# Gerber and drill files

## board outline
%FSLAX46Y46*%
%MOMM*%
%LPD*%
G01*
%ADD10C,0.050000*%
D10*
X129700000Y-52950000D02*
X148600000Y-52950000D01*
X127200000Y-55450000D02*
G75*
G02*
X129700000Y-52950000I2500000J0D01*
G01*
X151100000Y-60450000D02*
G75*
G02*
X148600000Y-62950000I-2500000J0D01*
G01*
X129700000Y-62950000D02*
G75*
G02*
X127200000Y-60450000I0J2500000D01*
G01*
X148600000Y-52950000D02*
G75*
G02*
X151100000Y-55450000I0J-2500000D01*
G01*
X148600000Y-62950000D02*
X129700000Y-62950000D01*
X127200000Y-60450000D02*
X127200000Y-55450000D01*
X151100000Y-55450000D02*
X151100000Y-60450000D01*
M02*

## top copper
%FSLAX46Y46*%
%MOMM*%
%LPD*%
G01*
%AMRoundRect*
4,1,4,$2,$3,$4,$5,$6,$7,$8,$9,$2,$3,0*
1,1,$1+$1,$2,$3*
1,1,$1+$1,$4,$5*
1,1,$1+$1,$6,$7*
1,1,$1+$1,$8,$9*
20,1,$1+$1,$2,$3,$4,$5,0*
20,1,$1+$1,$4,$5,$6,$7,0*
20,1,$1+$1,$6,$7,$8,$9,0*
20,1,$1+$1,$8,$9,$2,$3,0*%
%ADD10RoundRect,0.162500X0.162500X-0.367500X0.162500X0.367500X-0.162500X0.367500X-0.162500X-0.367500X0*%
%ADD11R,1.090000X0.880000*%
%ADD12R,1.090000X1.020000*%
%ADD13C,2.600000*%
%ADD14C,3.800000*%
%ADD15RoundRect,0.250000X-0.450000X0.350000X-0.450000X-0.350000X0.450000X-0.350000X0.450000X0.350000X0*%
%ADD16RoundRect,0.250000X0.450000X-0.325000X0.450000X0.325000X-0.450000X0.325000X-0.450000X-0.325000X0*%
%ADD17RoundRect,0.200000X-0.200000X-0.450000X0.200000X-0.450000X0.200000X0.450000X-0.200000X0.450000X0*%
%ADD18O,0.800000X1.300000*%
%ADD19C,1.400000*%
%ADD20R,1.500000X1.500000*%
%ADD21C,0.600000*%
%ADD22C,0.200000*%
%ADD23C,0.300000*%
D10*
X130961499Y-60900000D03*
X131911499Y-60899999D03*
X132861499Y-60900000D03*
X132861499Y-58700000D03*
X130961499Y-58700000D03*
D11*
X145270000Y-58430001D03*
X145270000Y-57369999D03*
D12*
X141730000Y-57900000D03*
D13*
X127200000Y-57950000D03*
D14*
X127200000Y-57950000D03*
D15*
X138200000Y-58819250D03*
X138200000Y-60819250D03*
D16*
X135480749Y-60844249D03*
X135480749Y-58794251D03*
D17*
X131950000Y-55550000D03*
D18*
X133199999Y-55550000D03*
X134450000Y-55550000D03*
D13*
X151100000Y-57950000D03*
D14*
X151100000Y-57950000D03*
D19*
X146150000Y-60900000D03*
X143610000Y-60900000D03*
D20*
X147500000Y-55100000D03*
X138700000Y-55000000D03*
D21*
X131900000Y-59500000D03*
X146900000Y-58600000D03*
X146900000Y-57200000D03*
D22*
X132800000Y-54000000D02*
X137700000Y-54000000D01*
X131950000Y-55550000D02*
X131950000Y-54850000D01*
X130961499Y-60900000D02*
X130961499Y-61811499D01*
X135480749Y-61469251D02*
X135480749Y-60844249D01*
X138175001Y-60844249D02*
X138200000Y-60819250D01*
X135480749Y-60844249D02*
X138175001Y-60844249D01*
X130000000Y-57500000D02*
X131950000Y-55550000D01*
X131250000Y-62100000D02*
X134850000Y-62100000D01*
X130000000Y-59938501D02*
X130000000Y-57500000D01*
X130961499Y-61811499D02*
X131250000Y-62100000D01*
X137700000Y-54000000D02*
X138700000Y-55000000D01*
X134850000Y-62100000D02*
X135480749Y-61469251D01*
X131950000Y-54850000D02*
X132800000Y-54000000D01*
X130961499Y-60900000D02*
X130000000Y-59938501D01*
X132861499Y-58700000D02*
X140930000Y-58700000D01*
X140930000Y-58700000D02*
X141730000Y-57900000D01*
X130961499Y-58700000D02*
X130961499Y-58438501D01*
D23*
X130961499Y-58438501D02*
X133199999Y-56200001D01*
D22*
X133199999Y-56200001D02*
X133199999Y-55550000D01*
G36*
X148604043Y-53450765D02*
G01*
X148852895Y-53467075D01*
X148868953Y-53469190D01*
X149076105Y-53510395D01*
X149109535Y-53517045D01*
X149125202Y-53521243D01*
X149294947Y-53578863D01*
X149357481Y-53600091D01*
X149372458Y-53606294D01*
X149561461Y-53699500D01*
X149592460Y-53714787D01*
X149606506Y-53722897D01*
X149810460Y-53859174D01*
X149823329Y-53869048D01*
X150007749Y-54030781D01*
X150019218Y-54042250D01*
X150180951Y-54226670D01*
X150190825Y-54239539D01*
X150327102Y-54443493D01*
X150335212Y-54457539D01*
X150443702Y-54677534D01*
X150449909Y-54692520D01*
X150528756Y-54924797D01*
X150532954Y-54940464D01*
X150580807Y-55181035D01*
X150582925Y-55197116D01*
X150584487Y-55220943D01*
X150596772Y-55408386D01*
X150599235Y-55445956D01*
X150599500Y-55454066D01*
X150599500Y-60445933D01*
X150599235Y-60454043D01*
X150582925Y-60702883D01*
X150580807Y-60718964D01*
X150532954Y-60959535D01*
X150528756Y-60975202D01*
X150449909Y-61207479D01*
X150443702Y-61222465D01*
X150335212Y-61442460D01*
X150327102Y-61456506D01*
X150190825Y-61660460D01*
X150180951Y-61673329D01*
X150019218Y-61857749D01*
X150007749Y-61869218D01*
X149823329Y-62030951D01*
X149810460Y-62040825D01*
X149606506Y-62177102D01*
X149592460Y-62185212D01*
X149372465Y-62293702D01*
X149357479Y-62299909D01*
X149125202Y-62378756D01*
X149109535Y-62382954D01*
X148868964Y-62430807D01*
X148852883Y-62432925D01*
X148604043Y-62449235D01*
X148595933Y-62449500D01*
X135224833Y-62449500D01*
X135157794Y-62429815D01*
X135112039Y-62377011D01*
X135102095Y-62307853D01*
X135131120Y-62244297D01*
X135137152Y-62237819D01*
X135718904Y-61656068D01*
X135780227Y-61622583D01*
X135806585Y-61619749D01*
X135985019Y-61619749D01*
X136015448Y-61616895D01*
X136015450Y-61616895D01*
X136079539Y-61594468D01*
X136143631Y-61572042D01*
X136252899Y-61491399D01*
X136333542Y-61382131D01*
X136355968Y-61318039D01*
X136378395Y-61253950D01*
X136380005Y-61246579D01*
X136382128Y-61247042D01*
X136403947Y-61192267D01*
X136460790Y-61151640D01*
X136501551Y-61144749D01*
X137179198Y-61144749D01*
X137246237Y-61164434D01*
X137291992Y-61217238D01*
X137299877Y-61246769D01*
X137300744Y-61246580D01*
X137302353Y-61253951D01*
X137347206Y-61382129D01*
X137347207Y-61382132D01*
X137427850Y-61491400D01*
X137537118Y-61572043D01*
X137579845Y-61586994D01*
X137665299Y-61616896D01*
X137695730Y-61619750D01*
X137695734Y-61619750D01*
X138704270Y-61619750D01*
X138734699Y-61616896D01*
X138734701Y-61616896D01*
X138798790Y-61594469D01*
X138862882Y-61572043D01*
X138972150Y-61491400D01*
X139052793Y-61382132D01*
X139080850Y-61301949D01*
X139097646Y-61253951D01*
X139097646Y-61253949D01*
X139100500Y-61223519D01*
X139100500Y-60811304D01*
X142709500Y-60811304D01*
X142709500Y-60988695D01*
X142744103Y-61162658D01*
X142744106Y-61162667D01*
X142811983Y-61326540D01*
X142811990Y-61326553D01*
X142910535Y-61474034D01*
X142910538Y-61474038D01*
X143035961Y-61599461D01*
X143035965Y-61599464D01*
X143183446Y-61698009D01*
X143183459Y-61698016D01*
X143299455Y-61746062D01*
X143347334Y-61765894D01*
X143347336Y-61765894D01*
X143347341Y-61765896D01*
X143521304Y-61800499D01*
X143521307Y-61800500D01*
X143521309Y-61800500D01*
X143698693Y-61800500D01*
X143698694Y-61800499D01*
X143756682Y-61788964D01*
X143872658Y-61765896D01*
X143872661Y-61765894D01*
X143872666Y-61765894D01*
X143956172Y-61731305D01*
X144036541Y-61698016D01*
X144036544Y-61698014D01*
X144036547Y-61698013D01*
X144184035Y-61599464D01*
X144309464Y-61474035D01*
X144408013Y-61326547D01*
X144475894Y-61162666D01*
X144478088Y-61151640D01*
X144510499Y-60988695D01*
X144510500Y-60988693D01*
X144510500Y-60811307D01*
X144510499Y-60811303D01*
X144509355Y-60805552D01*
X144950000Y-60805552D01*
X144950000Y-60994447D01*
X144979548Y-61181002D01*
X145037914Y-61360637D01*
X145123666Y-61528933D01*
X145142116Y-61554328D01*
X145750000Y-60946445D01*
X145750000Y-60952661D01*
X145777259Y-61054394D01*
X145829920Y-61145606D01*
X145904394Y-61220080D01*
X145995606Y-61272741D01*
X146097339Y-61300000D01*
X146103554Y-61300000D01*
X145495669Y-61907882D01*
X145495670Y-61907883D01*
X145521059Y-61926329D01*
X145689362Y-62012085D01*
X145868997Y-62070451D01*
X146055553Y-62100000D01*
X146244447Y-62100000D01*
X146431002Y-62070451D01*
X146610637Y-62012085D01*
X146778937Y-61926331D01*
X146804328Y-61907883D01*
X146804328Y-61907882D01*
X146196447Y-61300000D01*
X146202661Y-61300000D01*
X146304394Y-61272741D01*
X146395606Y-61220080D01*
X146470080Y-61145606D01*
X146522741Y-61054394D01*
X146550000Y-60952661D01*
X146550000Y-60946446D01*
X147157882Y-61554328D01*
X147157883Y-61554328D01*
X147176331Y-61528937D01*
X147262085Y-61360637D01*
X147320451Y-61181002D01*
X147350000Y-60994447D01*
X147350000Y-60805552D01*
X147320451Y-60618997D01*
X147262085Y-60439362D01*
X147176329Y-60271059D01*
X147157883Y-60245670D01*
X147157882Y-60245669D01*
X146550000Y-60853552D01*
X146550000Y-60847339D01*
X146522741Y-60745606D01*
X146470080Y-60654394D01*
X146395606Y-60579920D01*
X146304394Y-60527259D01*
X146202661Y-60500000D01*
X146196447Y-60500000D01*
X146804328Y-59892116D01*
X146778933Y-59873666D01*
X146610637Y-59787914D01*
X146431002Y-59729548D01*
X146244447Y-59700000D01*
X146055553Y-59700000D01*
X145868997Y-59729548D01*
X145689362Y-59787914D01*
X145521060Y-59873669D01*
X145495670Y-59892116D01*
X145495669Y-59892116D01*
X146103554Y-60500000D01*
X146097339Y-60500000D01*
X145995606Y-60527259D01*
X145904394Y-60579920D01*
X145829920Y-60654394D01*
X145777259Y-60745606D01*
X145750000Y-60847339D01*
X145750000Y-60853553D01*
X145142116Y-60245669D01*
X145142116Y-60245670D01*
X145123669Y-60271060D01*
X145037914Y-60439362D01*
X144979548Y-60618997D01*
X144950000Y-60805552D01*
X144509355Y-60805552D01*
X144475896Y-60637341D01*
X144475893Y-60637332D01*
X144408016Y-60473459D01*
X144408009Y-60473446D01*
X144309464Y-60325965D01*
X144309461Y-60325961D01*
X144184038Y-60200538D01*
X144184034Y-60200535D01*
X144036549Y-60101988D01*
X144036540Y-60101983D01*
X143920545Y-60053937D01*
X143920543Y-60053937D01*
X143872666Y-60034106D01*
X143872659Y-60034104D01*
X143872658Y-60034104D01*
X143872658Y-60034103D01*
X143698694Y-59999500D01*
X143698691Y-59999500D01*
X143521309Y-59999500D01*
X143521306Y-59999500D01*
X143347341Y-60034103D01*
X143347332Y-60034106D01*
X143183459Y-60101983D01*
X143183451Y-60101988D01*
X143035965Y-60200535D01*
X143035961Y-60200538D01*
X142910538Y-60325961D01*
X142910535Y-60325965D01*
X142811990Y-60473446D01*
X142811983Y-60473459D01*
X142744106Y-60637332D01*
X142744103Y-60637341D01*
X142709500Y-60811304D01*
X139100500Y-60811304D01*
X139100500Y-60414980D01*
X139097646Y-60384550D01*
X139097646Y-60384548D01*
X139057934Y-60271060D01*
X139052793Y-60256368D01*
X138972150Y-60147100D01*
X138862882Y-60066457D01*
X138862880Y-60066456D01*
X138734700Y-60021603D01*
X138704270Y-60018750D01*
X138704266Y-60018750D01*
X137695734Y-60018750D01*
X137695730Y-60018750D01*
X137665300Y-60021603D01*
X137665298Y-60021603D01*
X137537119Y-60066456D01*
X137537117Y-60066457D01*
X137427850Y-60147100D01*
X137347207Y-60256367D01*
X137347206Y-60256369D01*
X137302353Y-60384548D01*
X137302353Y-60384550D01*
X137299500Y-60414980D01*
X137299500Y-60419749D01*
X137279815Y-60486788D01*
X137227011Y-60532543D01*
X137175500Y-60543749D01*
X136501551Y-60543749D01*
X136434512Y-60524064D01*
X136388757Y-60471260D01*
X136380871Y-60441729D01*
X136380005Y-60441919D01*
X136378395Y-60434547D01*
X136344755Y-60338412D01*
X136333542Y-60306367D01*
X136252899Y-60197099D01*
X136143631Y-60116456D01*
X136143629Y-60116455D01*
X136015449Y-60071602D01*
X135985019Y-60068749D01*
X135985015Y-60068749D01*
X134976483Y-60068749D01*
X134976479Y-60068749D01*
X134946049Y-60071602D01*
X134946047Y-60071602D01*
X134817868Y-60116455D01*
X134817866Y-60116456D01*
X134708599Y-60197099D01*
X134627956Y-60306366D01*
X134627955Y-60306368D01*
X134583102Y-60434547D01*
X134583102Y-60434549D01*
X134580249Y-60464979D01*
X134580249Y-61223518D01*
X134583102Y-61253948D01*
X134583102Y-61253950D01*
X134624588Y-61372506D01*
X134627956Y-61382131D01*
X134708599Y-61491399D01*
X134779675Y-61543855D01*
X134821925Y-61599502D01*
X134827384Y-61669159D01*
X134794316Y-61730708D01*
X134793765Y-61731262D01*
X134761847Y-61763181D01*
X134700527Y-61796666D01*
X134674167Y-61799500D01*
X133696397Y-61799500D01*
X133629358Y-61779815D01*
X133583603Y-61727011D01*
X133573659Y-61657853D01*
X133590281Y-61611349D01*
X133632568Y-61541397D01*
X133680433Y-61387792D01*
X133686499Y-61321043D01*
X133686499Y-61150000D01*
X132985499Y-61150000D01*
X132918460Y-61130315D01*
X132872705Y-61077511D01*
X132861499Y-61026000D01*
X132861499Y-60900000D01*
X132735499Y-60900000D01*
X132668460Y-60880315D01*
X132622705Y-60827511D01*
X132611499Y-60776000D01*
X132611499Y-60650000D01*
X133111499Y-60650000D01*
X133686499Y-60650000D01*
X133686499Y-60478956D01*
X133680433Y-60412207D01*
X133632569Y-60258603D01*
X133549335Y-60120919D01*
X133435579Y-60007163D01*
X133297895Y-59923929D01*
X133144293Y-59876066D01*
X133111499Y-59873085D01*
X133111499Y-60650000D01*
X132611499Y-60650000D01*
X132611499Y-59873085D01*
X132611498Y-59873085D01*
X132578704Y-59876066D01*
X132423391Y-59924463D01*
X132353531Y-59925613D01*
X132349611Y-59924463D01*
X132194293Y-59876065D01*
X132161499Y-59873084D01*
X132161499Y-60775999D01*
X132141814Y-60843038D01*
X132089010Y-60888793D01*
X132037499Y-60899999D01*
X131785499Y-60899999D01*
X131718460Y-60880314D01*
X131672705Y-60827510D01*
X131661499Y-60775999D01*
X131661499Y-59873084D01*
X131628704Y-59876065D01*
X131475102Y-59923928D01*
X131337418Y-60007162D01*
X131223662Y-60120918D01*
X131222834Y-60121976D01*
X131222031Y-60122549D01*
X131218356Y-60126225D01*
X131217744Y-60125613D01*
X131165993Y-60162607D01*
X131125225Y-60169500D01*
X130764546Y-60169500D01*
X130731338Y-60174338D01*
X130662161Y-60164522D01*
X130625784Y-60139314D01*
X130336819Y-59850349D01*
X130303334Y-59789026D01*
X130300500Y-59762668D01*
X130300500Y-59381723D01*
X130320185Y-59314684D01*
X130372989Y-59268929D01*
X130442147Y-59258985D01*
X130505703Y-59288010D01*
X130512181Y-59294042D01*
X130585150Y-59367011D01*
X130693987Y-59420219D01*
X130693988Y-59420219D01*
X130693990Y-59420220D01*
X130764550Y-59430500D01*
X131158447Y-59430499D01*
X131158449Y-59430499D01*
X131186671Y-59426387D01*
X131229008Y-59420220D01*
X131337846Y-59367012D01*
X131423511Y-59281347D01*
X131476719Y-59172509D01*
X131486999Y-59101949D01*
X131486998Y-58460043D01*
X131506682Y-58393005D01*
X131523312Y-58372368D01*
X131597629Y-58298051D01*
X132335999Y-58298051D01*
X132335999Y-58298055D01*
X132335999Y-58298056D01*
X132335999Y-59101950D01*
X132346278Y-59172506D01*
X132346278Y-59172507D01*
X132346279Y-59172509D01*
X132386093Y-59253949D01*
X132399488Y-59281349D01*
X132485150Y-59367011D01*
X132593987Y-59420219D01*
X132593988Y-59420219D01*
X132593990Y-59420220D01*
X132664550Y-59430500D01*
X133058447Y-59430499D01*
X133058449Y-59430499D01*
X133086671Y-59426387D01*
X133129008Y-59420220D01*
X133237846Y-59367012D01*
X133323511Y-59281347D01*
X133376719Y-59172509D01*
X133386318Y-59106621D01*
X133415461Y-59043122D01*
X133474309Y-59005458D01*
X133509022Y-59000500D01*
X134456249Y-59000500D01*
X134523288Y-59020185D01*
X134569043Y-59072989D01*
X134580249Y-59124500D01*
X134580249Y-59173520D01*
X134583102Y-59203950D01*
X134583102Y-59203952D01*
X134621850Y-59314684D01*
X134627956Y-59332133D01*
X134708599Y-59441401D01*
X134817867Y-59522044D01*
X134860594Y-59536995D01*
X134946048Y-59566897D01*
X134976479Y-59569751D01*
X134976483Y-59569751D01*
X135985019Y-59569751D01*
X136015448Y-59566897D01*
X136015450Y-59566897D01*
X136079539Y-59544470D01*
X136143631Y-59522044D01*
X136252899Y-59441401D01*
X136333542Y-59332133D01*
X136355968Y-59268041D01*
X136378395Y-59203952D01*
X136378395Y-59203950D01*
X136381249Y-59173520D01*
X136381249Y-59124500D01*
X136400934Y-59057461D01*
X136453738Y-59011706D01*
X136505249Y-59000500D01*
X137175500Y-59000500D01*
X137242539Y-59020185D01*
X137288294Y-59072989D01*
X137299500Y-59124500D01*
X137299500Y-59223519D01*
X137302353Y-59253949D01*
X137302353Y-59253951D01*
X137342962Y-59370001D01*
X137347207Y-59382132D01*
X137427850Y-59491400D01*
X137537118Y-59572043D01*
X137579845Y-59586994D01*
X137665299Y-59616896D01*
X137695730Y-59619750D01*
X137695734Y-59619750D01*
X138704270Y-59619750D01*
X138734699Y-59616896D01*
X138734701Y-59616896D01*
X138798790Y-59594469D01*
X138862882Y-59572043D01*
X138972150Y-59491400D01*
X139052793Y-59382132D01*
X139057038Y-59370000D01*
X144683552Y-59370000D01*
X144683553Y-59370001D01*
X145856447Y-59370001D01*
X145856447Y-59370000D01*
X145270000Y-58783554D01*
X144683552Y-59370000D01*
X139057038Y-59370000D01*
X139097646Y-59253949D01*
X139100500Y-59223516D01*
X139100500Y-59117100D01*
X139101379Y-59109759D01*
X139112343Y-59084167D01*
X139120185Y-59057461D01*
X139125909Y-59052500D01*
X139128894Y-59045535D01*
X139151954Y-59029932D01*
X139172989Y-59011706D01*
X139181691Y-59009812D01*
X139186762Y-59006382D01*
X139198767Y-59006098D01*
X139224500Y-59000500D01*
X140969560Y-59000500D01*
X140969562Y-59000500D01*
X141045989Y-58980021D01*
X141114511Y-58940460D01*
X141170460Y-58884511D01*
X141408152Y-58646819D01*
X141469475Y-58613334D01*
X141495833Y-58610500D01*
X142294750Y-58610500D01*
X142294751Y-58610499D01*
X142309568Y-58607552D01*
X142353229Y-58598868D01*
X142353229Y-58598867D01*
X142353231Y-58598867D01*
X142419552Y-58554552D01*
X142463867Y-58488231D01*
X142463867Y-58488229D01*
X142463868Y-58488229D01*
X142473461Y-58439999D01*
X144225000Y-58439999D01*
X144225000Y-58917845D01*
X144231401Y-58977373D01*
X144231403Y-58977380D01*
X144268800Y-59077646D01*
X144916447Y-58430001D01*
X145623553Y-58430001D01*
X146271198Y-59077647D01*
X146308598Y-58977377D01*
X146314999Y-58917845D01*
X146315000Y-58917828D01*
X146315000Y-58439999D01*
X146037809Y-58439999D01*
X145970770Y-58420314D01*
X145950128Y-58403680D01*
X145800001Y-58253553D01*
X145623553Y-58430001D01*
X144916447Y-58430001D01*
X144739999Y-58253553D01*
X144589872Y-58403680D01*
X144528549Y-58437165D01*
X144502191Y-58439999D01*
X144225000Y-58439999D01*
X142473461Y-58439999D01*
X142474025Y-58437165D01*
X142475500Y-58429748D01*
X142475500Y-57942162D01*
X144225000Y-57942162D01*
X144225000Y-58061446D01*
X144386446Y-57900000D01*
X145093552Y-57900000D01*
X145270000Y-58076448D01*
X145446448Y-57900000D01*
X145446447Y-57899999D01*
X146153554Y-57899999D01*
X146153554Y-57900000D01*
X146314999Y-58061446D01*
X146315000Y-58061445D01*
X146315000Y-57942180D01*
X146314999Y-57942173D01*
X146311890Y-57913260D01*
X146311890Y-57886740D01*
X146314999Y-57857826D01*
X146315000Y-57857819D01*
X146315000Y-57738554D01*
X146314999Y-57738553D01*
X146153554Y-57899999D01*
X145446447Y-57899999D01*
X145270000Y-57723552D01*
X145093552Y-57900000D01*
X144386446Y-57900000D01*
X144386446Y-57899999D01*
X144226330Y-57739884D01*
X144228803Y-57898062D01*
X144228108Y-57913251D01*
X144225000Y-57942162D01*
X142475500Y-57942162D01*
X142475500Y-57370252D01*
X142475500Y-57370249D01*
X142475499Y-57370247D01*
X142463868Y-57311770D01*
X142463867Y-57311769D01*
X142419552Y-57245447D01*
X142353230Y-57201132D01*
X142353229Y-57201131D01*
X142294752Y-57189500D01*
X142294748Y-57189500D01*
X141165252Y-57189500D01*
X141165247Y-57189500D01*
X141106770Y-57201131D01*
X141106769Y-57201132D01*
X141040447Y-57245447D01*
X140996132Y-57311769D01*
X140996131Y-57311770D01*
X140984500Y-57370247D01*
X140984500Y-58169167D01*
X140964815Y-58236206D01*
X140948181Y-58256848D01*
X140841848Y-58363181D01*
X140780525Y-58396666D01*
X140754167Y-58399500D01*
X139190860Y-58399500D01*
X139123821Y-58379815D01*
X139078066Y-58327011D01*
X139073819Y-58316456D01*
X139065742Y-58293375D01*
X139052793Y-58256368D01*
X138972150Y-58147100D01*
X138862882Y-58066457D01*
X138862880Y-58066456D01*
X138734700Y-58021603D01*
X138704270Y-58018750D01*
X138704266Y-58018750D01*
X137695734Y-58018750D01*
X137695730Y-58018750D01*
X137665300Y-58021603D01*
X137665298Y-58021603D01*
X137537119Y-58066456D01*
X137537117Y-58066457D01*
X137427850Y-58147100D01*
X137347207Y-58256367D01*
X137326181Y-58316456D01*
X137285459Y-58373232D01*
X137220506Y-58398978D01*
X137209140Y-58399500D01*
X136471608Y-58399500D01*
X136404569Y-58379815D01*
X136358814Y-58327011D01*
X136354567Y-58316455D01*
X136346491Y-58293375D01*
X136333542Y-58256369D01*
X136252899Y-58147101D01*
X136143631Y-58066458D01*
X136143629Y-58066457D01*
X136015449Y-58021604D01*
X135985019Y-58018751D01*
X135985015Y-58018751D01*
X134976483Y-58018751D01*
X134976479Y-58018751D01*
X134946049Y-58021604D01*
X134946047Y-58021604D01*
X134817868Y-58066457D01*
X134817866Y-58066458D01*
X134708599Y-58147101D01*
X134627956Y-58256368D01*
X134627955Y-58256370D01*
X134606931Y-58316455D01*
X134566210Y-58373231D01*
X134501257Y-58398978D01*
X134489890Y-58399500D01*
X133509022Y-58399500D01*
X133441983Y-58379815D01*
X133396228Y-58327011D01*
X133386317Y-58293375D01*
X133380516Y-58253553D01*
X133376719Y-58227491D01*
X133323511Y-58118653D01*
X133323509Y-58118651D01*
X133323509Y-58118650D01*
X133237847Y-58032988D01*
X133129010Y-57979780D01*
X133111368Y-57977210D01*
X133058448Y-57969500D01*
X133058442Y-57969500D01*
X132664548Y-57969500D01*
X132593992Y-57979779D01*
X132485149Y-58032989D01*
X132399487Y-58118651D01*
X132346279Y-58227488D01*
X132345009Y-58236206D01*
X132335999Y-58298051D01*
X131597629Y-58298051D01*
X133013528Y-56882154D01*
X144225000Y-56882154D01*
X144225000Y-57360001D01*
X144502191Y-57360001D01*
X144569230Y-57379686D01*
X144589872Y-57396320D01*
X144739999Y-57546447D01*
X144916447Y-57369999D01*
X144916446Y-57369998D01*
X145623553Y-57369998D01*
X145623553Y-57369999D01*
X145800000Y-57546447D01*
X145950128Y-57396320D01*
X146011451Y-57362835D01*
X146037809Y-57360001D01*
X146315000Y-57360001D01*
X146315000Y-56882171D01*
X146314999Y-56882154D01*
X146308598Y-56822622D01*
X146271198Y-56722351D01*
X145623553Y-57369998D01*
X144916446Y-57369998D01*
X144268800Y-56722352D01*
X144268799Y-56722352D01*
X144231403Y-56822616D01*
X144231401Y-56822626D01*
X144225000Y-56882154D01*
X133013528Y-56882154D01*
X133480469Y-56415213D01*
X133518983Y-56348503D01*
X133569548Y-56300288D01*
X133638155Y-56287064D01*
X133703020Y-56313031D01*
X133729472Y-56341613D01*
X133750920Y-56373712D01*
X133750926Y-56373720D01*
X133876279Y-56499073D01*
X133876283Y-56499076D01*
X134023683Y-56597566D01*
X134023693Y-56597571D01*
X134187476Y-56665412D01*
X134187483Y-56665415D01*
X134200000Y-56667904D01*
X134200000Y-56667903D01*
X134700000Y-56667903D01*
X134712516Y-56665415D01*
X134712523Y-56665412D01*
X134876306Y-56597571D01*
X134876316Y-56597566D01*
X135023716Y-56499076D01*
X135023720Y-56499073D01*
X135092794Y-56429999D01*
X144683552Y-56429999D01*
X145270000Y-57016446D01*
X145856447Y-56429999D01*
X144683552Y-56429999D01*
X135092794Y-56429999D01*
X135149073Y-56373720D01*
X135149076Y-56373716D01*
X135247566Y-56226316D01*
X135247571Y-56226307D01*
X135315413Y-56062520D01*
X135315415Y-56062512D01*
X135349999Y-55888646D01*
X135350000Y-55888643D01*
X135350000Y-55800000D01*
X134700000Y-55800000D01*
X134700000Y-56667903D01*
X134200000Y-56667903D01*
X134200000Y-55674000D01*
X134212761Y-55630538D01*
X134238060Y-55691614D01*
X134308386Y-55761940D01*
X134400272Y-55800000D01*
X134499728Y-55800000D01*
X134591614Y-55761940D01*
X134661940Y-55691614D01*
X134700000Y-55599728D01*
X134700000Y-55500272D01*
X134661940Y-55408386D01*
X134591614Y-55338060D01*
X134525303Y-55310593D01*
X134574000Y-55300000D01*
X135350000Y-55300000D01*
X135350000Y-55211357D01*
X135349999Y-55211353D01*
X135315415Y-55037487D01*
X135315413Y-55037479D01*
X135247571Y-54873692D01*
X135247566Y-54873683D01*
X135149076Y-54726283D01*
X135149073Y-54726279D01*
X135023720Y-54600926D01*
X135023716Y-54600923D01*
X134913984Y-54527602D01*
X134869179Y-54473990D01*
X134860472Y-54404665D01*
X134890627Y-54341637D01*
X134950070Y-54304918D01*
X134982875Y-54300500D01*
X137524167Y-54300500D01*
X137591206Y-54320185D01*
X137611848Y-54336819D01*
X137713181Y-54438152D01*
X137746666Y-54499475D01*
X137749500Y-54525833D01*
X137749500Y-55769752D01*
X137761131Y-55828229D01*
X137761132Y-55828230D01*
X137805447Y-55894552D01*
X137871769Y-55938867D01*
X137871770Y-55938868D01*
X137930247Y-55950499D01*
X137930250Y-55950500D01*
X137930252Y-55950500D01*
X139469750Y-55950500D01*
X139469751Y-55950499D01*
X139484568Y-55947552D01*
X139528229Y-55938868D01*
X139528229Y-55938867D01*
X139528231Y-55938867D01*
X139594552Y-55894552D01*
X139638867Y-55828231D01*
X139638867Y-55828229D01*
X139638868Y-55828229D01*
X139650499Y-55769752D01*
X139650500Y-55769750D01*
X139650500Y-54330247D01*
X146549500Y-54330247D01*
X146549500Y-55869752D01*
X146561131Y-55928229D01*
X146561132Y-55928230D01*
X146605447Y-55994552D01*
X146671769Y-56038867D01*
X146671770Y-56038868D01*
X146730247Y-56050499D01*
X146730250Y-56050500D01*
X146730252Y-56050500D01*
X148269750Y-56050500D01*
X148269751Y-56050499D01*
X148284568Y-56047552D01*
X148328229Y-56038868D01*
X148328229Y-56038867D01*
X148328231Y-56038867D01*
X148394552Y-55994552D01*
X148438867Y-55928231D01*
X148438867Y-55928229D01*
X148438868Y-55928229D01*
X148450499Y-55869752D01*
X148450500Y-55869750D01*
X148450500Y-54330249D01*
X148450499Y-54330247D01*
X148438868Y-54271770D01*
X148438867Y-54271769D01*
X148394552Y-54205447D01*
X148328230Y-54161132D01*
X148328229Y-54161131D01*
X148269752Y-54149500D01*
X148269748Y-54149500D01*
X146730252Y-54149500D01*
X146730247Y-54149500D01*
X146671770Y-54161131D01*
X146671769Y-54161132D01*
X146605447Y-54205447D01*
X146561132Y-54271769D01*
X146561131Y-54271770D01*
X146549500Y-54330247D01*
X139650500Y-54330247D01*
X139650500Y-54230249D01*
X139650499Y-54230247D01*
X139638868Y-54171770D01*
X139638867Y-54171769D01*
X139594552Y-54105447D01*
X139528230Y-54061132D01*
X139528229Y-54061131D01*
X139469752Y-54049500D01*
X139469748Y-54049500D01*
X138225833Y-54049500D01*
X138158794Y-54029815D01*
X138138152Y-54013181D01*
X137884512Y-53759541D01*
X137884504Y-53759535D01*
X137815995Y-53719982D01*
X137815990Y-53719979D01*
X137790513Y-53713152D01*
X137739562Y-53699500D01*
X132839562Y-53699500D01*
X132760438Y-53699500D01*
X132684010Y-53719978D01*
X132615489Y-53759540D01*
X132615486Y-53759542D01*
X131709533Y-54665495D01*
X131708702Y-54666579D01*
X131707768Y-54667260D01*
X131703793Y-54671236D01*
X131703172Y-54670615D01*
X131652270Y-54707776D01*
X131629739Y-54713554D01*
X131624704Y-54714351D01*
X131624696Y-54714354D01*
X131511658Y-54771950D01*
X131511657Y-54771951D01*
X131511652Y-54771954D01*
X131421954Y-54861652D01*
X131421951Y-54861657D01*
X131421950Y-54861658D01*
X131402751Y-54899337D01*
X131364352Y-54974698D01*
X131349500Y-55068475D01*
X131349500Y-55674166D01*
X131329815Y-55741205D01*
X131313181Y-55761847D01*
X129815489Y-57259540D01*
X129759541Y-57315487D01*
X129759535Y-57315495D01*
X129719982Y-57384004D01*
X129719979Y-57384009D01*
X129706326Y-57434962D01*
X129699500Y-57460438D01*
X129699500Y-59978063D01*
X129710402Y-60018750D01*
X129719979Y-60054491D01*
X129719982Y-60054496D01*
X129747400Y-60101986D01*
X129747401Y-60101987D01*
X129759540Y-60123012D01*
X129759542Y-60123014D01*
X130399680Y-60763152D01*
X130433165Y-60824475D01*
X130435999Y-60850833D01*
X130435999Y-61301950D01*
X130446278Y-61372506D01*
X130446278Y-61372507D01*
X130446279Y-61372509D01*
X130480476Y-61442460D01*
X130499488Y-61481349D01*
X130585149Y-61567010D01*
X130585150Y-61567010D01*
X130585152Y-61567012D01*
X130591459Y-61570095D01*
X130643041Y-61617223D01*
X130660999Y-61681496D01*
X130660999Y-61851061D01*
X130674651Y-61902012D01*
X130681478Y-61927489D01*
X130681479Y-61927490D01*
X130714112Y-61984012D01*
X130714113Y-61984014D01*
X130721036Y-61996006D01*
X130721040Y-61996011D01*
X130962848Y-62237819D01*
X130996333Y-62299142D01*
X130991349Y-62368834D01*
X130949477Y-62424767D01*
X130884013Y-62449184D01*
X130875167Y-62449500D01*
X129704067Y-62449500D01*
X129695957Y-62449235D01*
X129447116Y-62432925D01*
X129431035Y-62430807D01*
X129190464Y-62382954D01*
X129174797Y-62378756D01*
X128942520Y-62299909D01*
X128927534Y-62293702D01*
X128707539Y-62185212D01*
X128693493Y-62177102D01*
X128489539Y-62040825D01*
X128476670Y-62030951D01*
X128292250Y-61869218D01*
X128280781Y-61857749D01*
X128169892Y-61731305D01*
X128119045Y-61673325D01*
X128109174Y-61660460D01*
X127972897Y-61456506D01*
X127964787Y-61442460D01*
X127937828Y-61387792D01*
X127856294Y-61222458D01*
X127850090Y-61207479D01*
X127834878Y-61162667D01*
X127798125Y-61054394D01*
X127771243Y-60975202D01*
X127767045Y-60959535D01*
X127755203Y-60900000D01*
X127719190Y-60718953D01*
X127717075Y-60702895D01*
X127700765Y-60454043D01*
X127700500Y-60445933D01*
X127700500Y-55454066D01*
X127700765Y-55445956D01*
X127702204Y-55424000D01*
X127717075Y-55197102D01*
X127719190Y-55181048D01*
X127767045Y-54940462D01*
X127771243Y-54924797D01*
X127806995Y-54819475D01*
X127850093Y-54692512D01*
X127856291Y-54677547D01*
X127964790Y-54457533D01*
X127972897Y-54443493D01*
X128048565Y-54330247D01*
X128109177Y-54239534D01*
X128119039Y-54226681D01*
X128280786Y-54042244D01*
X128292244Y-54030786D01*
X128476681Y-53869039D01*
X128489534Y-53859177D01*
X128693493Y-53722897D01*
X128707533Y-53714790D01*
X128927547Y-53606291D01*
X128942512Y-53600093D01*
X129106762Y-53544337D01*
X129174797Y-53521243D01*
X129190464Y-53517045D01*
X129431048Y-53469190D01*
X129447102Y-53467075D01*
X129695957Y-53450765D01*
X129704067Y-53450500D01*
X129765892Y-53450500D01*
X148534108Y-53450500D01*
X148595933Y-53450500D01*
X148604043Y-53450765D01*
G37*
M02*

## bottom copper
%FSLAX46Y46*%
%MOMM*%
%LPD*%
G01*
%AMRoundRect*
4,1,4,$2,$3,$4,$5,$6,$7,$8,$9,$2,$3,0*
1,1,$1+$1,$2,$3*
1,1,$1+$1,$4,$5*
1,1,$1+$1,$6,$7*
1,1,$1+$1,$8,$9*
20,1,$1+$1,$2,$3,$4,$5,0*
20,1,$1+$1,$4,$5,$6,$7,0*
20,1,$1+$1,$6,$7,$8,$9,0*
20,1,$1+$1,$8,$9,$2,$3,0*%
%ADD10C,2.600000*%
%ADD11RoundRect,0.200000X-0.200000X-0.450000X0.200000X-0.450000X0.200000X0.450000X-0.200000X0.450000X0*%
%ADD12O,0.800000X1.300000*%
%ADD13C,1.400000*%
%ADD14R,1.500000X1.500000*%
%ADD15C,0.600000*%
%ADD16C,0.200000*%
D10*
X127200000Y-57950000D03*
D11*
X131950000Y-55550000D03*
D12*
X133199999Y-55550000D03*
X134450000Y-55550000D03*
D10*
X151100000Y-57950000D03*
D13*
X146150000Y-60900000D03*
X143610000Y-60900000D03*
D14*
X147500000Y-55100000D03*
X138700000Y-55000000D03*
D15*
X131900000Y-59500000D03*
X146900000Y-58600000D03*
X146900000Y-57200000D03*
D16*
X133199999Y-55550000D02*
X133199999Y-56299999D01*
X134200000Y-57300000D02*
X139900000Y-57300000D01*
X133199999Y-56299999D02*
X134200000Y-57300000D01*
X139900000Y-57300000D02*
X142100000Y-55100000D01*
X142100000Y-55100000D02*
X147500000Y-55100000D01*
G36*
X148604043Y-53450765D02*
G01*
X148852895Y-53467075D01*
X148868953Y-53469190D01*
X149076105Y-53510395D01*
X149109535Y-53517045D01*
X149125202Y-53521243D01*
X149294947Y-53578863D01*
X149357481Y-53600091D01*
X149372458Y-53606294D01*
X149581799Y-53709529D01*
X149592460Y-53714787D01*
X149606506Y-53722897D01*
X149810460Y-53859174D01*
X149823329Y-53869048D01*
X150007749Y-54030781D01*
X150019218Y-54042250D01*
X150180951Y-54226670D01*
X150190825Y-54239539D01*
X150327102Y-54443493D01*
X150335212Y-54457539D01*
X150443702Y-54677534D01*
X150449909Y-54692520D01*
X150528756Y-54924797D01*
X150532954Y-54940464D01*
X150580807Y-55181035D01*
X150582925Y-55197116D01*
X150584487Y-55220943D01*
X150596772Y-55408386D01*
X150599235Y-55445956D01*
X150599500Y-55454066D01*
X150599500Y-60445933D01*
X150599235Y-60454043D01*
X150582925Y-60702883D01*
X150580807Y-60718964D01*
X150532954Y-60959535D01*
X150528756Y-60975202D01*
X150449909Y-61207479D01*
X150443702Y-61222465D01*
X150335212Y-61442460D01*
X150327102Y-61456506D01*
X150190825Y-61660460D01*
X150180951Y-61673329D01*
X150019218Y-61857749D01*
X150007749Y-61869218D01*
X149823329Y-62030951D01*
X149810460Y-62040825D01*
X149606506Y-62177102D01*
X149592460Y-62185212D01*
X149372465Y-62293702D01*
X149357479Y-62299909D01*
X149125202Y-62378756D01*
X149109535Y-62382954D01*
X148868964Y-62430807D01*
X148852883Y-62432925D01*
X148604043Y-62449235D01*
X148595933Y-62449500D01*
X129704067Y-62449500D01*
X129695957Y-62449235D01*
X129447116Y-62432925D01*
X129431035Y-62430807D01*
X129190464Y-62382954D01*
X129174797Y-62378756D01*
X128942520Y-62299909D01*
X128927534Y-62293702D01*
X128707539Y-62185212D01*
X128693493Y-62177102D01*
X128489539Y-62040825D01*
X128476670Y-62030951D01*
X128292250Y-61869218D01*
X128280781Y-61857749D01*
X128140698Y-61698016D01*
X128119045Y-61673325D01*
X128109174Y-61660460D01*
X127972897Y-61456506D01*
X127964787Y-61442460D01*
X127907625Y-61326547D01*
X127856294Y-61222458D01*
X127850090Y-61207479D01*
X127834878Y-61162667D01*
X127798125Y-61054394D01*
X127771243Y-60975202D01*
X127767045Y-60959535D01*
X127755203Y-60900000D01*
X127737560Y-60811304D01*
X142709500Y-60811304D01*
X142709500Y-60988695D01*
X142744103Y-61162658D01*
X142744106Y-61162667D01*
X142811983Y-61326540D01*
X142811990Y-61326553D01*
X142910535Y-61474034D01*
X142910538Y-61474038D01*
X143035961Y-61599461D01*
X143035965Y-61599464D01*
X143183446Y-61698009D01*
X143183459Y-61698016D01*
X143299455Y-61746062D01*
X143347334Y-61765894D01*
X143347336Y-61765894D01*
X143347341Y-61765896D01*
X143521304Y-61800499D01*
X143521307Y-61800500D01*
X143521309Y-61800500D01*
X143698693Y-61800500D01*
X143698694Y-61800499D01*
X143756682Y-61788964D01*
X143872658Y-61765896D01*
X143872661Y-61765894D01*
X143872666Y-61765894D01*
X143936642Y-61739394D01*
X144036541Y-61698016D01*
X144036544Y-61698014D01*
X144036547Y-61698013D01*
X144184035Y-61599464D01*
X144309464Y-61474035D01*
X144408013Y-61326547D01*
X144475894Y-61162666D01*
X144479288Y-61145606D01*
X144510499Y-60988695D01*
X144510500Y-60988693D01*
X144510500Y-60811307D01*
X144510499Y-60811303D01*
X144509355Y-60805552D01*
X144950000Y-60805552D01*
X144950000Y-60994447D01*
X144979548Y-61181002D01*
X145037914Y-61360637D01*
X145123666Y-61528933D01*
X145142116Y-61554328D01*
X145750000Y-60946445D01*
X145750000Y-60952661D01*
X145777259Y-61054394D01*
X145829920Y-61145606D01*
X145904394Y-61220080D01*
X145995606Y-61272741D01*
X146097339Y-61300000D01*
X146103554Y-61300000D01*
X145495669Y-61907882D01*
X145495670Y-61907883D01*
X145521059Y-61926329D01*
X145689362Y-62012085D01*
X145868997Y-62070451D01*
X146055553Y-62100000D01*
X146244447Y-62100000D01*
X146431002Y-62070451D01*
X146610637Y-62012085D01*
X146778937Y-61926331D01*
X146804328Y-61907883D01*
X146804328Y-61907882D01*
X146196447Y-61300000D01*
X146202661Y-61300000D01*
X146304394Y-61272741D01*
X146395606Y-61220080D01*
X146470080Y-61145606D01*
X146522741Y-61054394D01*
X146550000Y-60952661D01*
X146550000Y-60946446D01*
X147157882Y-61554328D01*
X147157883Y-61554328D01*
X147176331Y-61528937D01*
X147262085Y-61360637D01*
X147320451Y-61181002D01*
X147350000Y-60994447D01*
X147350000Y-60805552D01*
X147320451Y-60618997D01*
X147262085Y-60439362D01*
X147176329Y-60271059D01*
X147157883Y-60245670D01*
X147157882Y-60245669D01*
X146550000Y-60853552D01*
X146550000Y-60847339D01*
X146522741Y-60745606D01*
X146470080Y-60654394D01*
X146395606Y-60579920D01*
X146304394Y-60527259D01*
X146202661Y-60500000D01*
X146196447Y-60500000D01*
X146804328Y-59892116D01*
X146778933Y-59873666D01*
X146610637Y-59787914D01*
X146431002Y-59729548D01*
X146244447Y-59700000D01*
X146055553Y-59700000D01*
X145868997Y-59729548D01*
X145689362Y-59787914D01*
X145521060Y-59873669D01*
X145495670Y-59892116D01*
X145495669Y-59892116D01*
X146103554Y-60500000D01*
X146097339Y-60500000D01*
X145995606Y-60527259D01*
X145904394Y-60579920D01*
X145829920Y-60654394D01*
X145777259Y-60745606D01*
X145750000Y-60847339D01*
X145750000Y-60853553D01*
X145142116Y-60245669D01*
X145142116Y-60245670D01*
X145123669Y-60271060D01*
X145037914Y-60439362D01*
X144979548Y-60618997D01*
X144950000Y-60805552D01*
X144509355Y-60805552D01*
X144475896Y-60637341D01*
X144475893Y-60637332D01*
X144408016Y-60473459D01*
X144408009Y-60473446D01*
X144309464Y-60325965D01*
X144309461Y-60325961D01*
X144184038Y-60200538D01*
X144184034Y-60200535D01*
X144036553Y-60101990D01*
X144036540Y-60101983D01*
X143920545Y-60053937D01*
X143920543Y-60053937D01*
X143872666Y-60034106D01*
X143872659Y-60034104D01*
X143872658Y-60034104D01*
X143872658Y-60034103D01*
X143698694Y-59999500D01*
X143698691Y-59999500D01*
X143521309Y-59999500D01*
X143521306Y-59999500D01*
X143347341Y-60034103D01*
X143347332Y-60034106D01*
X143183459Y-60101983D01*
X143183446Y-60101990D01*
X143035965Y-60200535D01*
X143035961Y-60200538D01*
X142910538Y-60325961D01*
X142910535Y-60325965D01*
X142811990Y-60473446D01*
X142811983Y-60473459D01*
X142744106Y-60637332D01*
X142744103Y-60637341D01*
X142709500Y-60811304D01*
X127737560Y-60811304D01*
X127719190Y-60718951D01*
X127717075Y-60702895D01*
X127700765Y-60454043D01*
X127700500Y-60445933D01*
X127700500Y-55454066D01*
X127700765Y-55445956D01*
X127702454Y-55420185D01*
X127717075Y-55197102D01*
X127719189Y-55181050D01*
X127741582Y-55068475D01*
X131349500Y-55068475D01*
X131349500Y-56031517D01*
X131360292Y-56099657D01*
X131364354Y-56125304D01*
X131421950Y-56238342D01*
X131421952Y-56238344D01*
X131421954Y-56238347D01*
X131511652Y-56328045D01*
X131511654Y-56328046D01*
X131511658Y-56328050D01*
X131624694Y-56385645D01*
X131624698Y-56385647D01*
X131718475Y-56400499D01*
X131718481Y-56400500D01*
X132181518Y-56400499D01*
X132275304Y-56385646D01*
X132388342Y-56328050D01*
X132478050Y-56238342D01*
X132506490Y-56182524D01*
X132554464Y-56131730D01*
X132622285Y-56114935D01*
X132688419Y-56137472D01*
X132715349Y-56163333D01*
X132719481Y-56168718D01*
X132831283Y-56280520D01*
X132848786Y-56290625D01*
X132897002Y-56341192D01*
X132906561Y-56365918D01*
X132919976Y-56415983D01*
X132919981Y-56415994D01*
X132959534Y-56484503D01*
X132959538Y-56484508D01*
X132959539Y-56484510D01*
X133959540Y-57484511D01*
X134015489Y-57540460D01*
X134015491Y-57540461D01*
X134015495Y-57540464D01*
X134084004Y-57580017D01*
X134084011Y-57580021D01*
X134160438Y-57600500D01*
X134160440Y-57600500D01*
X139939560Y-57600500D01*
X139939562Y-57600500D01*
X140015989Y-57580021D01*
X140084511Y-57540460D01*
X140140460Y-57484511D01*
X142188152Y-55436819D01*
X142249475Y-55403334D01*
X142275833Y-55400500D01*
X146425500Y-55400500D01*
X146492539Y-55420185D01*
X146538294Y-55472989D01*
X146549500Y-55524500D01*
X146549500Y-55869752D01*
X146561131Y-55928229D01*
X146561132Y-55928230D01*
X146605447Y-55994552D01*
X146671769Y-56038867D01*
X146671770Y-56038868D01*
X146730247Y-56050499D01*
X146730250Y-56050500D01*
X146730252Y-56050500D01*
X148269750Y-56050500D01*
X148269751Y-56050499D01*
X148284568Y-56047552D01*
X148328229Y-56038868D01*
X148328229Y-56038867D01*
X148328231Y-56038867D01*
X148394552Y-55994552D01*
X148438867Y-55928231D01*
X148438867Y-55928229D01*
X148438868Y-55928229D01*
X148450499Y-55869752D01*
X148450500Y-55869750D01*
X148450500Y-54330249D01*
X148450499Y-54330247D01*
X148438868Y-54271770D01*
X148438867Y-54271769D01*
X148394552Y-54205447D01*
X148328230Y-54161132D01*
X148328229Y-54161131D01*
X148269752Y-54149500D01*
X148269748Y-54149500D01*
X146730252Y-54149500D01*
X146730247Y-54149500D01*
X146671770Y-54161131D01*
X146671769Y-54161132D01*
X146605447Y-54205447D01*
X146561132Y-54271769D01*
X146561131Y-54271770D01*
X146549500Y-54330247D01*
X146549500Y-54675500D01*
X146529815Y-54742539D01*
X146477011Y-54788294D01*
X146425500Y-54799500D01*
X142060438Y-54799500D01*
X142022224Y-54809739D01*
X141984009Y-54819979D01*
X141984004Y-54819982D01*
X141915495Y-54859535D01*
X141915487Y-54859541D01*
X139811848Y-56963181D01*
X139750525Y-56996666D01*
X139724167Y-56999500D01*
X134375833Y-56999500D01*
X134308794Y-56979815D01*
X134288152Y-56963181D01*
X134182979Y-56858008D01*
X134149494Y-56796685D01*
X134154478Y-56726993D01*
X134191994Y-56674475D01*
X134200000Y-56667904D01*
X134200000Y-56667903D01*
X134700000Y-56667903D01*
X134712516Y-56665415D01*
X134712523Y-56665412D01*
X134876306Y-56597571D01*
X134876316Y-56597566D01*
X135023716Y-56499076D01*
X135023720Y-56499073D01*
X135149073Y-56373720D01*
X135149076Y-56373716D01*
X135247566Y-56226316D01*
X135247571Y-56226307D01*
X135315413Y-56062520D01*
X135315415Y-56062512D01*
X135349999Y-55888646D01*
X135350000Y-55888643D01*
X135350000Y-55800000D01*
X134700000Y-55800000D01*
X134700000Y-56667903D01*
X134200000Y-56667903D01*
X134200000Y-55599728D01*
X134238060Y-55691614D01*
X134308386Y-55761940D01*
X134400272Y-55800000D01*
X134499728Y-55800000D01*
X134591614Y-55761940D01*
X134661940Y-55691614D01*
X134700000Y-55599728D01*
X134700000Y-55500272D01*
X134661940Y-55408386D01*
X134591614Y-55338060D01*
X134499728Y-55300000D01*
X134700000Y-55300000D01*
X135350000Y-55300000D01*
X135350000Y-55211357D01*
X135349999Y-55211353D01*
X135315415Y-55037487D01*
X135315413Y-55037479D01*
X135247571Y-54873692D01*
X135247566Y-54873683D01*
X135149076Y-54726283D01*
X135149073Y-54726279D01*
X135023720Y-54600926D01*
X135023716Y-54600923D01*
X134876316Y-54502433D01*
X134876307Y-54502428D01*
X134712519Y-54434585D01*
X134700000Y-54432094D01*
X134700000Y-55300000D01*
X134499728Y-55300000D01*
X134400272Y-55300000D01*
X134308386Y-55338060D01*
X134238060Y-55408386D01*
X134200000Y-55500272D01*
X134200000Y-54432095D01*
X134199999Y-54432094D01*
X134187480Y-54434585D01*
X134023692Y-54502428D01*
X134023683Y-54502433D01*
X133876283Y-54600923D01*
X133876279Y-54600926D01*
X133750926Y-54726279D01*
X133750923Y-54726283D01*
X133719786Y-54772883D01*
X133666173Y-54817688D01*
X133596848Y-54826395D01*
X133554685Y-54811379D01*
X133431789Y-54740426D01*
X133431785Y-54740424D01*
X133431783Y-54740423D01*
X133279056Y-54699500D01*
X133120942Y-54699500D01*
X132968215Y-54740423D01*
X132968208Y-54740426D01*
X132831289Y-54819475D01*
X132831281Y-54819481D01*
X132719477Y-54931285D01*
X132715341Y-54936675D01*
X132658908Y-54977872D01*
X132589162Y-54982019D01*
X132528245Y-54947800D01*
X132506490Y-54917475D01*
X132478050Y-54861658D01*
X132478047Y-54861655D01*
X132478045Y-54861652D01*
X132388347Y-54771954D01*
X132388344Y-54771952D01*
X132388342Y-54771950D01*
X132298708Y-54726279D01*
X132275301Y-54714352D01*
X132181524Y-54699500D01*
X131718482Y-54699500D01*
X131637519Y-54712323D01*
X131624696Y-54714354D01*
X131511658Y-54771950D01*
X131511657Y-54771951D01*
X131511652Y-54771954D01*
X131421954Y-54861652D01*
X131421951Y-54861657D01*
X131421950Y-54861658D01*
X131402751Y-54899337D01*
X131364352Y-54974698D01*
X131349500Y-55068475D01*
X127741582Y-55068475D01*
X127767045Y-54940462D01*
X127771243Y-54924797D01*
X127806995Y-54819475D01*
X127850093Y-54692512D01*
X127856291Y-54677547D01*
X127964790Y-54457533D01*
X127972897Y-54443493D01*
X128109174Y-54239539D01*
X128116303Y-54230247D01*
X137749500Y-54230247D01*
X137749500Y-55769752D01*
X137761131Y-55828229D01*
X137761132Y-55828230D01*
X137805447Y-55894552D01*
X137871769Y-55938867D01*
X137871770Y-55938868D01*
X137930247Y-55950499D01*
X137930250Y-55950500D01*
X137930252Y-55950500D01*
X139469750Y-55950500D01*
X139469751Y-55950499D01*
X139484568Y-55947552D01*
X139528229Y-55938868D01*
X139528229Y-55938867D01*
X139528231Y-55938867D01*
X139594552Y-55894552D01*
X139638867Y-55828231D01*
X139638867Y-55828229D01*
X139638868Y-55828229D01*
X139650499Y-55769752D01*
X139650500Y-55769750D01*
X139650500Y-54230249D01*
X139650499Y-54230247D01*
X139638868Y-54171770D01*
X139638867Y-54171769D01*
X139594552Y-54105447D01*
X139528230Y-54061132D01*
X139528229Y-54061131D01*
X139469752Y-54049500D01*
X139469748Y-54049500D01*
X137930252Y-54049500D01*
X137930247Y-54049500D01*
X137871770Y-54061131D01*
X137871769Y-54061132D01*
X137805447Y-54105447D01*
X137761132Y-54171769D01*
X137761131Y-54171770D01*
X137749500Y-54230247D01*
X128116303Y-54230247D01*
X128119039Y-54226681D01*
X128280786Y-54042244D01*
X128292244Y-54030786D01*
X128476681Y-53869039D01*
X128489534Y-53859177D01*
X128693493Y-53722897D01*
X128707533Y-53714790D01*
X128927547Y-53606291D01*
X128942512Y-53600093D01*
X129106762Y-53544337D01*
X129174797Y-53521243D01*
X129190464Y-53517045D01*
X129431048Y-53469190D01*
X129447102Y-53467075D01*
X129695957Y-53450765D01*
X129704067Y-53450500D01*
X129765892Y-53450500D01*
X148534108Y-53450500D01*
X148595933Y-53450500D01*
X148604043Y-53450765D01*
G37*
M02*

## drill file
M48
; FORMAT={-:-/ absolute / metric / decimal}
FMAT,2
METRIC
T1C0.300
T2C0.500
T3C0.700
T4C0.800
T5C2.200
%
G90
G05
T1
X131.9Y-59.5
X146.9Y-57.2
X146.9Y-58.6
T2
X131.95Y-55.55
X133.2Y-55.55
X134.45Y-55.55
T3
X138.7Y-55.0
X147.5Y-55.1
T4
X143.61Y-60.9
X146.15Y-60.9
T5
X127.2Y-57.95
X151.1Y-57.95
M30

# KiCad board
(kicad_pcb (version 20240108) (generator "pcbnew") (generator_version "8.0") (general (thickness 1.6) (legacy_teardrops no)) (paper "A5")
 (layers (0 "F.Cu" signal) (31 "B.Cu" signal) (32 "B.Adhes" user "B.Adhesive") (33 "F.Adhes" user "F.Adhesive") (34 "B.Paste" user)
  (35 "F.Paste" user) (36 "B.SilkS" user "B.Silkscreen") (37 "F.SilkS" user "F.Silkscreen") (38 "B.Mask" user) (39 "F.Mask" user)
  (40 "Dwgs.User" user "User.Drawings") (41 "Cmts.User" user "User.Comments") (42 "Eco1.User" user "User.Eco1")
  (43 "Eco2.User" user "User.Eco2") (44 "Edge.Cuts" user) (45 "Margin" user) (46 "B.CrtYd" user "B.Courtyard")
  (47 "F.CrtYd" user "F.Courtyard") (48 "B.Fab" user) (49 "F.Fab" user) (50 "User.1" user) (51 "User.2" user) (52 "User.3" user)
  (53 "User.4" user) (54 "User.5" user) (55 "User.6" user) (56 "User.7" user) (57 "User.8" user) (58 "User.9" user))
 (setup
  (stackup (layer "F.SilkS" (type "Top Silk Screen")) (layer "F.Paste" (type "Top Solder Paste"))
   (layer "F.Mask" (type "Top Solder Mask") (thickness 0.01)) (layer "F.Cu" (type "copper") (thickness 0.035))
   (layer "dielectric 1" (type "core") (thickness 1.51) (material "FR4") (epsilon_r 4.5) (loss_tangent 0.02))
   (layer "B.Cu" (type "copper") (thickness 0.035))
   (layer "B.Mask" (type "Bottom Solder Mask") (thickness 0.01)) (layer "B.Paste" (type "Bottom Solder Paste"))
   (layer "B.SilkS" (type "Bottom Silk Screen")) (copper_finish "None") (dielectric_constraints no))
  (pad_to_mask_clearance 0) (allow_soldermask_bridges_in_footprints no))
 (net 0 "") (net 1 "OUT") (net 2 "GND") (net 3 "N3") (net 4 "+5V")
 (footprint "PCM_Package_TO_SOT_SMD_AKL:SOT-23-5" (layer "F.Cu") (at 131.911499 59.8 90)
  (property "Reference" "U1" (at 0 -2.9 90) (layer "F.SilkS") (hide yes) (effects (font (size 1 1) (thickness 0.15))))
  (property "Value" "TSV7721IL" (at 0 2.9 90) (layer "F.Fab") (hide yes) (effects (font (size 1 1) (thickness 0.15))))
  (pad "1" smd roundrect (at -1.1 -0.95 90) (size 1.06 0.65) (layers "F.Cu" "F.Paste" "F.Mask") (roundrect_rratio 0.25) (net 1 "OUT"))
  (pad "2" smd roundrect (at -1.099999 0 90) (size 1.06 0.65) (layers "F.Cu" "F.Paste" "F.Mask") (roundrect_rratio 0.25) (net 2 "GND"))
  (pad "3" smd roundrect (at -1.1 0.95 90) (size 1.06 0.65) (layers "F.Cu" "F.Paste" "F.Mask") (roundrect_rratio 0.25) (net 2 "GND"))
  (pad "4" smd roundrect (at 1.1 0.95 90) (size 1.06 0.65) (layers "F.Cu" "F.Paste" "F.Mask") (roundrect_rratio 0.25) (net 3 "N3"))
  (pad "5" smd roundrect (at 1.1 -0.95 90) (size 1.06 0.65) (layers "F.Cu" "F.Paste" "F.Mask") (roundrect_rratio 0.25) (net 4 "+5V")))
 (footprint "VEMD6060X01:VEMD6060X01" (layer "F.Cu") (at 143.5 57.9 180)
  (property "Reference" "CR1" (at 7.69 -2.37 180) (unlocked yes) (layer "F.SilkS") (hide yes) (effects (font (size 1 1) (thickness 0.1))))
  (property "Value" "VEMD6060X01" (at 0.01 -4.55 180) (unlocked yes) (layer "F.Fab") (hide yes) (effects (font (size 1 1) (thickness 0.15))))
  (pad "1" smd rect (at -1.77 -0.530001 180) (size 1.09 0.88) (layers "F.Cu" "F.Paste" "F.Mask") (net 2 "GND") (thermal_bridge_angle 45))
  (pad "2" smd rect (at -1.77 0.530001 180) (size 1.09 0.88) (layers "F.Cu" "F.Paste" "F.Mask") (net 2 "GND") (thermal_bridge_angle 45))
  (pad "3" smd rect (at 1.77 0 180) (size 1.09 1.02) (layers "F.Cu" "F.Paste" "F.Mask") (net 3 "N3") (thermal_bridge_angle 45)))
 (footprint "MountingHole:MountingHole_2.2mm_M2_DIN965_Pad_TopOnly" (layer "F.Cu") (at 127.2 57.95)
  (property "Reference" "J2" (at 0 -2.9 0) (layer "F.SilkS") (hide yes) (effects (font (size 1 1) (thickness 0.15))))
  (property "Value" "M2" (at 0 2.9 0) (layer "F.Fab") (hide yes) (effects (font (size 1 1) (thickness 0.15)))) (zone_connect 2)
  (pad "1" thru_hole circle (at 0 0) (size 2.6 2.6) (drill 2.2) (layers "*.Cu" "*.Mask") (remove_unused_layers no) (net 2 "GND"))
  (pad "1" connect circle (at 0 0) (size 3.8 3.8) (layers "F.Cu" "F.Mask") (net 2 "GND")))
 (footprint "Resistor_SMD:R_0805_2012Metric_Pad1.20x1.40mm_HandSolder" (layer "F.Cu") (at 138.2 59.81925 -90)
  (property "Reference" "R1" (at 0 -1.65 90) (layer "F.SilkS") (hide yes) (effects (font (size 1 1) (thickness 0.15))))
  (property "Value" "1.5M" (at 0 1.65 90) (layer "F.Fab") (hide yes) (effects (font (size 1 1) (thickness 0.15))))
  (pad "1" smd roundrect (at -1 0 270) (size 1.2 1.4) (layers "F.Cu" "F.Paste" "F.Mask") (roundrect_rratio 0.208333) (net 3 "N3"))
  (pad "2" smd roundrect (at 1 0 270) (size 1.2 1.4) (layers "F.Cu" "F.Paste" "F.Mask") (roundrect_rratio 0.208333) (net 1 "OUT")))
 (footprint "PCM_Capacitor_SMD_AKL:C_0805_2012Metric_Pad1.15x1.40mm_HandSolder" (layer "F.Cu") (at 135.480749 59.81925 90)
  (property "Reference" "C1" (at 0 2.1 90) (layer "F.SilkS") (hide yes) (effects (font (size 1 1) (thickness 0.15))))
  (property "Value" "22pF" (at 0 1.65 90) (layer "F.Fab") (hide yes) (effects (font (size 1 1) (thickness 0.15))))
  (pad "1" smd roundrect (at -1.024999 0 90) (size 1.15 1.4) (layers "F.Cu" "F.Paste" "F.Mask") (roundrect_rratio 0.217391) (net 1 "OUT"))
  (pad "2" smd roundrect (at 1.024999 0 90) (size 1.15 1.4) (layers "F.Cu" "F.Paste" "F.Mask") (roundrect_rratio 0.217391) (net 3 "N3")))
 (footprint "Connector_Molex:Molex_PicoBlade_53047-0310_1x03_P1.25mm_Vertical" (layer "F.Cu") (at 131.95 55.55)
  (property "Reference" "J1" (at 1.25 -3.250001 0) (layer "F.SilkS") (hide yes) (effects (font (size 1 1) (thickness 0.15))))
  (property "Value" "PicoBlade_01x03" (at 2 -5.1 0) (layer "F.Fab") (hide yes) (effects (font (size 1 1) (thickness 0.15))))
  (pad "1" thru_hole roundrect (at 0 0) (size 0.8 1.3) (drill 0.5) (layers "*.Cu" "*.Mask") (remove_unused_layers no)
   (roundrect_rratio 0.25) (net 1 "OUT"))
  (pad "2" thru_hole oval (at 1.249999 0) (size 0.8 1.3) (drill 0.5) (layers "*.Cu" "*.Mask") (remove_unused_layers no) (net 4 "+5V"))
  (pad "3" thru_hole oval (at 2.5 0) (size 0.8 1.3) (drill 0.5) (layers "*.Cu" "*.Mask") (remove_unused_layers no) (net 2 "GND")))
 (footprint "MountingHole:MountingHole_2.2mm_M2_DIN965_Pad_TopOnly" (layer "F.Cu") (at 151.1 57.95)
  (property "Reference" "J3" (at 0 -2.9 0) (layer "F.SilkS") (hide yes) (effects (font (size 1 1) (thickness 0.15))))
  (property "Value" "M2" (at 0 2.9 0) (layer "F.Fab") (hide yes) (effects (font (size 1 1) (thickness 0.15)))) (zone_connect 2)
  (pad "1" thru_hole circle (at 0 0) (size 2.6 2.6) (drill 2.2) (layers "*.Cu" "*.Mask") (remove_unused_layers no) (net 2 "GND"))
  (pad "1" connect circle (at 0 0) (size 3.8 3.8) (layers "F.Cu" "F.Mask") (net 2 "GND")))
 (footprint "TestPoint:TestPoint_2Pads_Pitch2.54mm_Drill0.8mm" (layer "B.Cu") (at 146.15 60.9 180)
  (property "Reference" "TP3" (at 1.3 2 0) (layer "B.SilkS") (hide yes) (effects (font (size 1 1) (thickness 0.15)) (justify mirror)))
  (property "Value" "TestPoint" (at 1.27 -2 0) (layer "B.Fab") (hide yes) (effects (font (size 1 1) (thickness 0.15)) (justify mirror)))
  (pad "1" thru_hole circle (at 0 0 180) (size 1.4 1.4) (drill 0.8) (layers "*.Cu" "*.Mask") (remove_unused_layers no) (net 2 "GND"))
  (pad "2" thru_hole circle (at 2.54 0 180) (size 1.4 1.4) (drill 0.8) (layers "*.Cu" "*.Mask") (remove_unused_layers no)))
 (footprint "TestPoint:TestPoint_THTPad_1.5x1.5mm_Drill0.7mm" (layer "B.Cu") (at 147.5 55.1 180)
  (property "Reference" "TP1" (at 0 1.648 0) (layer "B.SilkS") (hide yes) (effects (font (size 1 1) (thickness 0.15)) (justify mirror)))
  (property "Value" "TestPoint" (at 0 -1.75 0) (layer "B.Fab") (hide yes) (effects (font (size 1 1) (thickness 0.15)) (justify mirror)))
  (pad "1" thru_hole rect (at 0 0 180) (size 1.5 1.5) (drill 0.7) (layers "*.Cu" "*.Mask") (remove_unused_layers no) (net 4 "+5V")))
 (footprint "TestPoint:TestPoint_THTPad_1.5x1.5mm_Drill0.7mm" (layer "B.Cu") (at 138.7 55 180)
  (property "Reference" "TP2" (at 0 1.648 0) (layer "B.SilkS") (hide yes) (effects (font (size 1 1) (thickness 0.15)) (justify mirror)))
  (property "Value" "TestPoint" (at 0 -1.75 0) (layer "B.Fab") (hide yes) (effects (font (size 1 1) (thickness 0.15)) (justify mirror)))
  (pad "1" thru_hole rect (at 0 0 180) (size 1.5 1.5) (drill 0.7) (layers "*.Cu" "*.Mask") (remove_unused_layers no) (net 1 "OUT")))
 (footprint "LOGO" (layer "B.Cu") (at 139.13435 57.9 180)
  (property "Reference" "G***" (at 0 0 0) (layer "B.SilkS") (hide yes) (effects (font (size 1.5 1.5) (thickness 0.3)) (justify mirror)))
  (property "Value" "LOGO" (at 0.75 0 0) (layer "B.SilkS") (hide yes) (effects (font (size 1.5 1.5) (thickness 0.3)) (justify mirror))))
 (gr_line (start 129.7 52.95) (end 148.6 52.95) (stroke (width 0.05) (type default)) (layer "Edge.Cuts"))
 (gr_arc (start 127.2 55.45) (mid 127.932233 53.682233) (end 129.7 52.95) (stroke (width 0.05) (type default)) (layer "Edge.Cuts"))
 (gr_arc (start 151.1 60.45) (mid 150.367767 62.217767) (end 148.6 62.95) (stroke (width 0.05) (type default)) (layer "Edge.Cuts"))
 (gr_arc (start 129.7 62.95) (mid 127.932233 62.217767) (end 127.2 60.45) (stroke (width 0.05) (type default)) (layer "Edge.Cuts"))
 (gr_arc (start 148.6 52.95) (mid 150.367767 53.682233) (end 151.1 55.45) (stroke (width 0.05) (type default)) (layer "Edge.Cuts"))
 (gr_line (start 148.6 62.95) (end 129.7 62.95) (stroke (width 0.05) (type default)) (layer "Edge.Cuts"))
 (gr_line (start 127.2 60.45) (end 127.2 55.45) (stroke (width 0.05) (type default)) (layer "Edge.Cuts"))
 (gr_line (start 151.1 55.45) (end 151.1 60.45) (stroke (width 0.05) (type default)) (layer "Edge.Cuts"))
 (segment (start 132.8 54) (end 137.7 54) (width 0.2) (layer "F.Cu") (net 1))
 (segment (start 131.95 55.55) (end 131.95 54.85) (width 0.2) (layer "F.Cu") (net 1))
 (segment (start 130.961499 60.9) (end 130.961499 61.811499) (width 0.2) (layer "F.Cu") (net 1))
 (segment (start 135.480749 61.469251) (end 135.480749 60.844249) (width 0.2) (layer "F.Cu") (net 1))
 (segment (start 138.175001 60.844249) (end 138.2 60.81925) (width 0.2) (layer "F.Cu") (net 1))
 (segment (start 135.480749 60.844249) (end 138.175001 60.844249) (width 0.2) (layer "F.Cu") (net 1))
 (segment (start 130 57.5) (end 131.95 55.55) (width 0.2) (layer "F.Cu") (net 1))
 (segment (start 131.25 62.1) (end 134.85 62.1) (width 0.2) (layer "F.Cu") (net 1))
 (segment (start 130 59.938501) (end 130 57.5) (width 0.2) (layer "F.Cu") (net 1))
 (segment (start 130.961499 61.811499) (end 131.25 62.1) (width 0.2) (layer "F.Cu") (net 1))
 (segment (start 137.7 54) (end 138.7 55) (width 0.2) (layer "F.Cu") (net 1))
 (segment (start 134.85 62.1) (end 135.480749 61.469251) (width 0.2) (layer "F.Cu") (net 1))
 (segment (start 131.95 54.85) (end 132.8 54) (width 0.2) (layer "F.Cu") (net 1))
 (segment (start 130.961499 60.9) (end 130 59.938501) (width 0.2) (layer "F.Cu") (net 1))
 (segment (start 132.861499 58.7) (end 140.93 58.7) (width 0.2) (layer "F.Cu") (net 3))
 (segment (start 140.93 58.7) (end 141.73 57.9) (width 0.2) (layer "F.Cu") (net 3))
 (via (at 131.9 59.5) (size 0.6) (drill 0.3) (layers "F.Cu" "B.Cu") (free yes) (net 2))
 (via (at 146.9 58.6) (size 0.6) (drill 0.3) (layers "F.Cu" "B.Cu") (free yes) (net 2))
 (via (at 146.9 57.2) (size 0.6) (drill 0.3) (layers "F.Cu" "B.Cu") (free yes) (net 2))
 (segment (start 130.961499 58.7) (end 130.961499 58.438501) (width 0.2) (layer "F.Cu") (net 4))
 (segment (start 130.961499 58.438501) (end 133.199999 56.200001) (width 0.3) (layer "F.Cu") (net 4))
 (segment (start 133.199999 56.200001) (end 133.199999 55.55) (width 0.2) (layer "F.Cu") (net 4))
 (segment (start 133.199999 55.55) (end 133.199999 56.299999) (width 0.2) (layer "B.Cu") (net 4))
 (segment (start 134.2 57.3) (end 139.9 57.3) (width 0.2) (layer "B.Cu") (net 4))
 (segment (start 133.199999 56.299999) (end 134.2 57.3) (width 0.2) (layer "B.Cu") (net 4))
 (segment (start 139.9 57.3) (end 142.1 55.1) (width 0.2) (layer "B.Cu") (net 4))
 (segment (start 142.1 55.1) (end 147.5 55.1) (width 0.2) (layer "B.Cu") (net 4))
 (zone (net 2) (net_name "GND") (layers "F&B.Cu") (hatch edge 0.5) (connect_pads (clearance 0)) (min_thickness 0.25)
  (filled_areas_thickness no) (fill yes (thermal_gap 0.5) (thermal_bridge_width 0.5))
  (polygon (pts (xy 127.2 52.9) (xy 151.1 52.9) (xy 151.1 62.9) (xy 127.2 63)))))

